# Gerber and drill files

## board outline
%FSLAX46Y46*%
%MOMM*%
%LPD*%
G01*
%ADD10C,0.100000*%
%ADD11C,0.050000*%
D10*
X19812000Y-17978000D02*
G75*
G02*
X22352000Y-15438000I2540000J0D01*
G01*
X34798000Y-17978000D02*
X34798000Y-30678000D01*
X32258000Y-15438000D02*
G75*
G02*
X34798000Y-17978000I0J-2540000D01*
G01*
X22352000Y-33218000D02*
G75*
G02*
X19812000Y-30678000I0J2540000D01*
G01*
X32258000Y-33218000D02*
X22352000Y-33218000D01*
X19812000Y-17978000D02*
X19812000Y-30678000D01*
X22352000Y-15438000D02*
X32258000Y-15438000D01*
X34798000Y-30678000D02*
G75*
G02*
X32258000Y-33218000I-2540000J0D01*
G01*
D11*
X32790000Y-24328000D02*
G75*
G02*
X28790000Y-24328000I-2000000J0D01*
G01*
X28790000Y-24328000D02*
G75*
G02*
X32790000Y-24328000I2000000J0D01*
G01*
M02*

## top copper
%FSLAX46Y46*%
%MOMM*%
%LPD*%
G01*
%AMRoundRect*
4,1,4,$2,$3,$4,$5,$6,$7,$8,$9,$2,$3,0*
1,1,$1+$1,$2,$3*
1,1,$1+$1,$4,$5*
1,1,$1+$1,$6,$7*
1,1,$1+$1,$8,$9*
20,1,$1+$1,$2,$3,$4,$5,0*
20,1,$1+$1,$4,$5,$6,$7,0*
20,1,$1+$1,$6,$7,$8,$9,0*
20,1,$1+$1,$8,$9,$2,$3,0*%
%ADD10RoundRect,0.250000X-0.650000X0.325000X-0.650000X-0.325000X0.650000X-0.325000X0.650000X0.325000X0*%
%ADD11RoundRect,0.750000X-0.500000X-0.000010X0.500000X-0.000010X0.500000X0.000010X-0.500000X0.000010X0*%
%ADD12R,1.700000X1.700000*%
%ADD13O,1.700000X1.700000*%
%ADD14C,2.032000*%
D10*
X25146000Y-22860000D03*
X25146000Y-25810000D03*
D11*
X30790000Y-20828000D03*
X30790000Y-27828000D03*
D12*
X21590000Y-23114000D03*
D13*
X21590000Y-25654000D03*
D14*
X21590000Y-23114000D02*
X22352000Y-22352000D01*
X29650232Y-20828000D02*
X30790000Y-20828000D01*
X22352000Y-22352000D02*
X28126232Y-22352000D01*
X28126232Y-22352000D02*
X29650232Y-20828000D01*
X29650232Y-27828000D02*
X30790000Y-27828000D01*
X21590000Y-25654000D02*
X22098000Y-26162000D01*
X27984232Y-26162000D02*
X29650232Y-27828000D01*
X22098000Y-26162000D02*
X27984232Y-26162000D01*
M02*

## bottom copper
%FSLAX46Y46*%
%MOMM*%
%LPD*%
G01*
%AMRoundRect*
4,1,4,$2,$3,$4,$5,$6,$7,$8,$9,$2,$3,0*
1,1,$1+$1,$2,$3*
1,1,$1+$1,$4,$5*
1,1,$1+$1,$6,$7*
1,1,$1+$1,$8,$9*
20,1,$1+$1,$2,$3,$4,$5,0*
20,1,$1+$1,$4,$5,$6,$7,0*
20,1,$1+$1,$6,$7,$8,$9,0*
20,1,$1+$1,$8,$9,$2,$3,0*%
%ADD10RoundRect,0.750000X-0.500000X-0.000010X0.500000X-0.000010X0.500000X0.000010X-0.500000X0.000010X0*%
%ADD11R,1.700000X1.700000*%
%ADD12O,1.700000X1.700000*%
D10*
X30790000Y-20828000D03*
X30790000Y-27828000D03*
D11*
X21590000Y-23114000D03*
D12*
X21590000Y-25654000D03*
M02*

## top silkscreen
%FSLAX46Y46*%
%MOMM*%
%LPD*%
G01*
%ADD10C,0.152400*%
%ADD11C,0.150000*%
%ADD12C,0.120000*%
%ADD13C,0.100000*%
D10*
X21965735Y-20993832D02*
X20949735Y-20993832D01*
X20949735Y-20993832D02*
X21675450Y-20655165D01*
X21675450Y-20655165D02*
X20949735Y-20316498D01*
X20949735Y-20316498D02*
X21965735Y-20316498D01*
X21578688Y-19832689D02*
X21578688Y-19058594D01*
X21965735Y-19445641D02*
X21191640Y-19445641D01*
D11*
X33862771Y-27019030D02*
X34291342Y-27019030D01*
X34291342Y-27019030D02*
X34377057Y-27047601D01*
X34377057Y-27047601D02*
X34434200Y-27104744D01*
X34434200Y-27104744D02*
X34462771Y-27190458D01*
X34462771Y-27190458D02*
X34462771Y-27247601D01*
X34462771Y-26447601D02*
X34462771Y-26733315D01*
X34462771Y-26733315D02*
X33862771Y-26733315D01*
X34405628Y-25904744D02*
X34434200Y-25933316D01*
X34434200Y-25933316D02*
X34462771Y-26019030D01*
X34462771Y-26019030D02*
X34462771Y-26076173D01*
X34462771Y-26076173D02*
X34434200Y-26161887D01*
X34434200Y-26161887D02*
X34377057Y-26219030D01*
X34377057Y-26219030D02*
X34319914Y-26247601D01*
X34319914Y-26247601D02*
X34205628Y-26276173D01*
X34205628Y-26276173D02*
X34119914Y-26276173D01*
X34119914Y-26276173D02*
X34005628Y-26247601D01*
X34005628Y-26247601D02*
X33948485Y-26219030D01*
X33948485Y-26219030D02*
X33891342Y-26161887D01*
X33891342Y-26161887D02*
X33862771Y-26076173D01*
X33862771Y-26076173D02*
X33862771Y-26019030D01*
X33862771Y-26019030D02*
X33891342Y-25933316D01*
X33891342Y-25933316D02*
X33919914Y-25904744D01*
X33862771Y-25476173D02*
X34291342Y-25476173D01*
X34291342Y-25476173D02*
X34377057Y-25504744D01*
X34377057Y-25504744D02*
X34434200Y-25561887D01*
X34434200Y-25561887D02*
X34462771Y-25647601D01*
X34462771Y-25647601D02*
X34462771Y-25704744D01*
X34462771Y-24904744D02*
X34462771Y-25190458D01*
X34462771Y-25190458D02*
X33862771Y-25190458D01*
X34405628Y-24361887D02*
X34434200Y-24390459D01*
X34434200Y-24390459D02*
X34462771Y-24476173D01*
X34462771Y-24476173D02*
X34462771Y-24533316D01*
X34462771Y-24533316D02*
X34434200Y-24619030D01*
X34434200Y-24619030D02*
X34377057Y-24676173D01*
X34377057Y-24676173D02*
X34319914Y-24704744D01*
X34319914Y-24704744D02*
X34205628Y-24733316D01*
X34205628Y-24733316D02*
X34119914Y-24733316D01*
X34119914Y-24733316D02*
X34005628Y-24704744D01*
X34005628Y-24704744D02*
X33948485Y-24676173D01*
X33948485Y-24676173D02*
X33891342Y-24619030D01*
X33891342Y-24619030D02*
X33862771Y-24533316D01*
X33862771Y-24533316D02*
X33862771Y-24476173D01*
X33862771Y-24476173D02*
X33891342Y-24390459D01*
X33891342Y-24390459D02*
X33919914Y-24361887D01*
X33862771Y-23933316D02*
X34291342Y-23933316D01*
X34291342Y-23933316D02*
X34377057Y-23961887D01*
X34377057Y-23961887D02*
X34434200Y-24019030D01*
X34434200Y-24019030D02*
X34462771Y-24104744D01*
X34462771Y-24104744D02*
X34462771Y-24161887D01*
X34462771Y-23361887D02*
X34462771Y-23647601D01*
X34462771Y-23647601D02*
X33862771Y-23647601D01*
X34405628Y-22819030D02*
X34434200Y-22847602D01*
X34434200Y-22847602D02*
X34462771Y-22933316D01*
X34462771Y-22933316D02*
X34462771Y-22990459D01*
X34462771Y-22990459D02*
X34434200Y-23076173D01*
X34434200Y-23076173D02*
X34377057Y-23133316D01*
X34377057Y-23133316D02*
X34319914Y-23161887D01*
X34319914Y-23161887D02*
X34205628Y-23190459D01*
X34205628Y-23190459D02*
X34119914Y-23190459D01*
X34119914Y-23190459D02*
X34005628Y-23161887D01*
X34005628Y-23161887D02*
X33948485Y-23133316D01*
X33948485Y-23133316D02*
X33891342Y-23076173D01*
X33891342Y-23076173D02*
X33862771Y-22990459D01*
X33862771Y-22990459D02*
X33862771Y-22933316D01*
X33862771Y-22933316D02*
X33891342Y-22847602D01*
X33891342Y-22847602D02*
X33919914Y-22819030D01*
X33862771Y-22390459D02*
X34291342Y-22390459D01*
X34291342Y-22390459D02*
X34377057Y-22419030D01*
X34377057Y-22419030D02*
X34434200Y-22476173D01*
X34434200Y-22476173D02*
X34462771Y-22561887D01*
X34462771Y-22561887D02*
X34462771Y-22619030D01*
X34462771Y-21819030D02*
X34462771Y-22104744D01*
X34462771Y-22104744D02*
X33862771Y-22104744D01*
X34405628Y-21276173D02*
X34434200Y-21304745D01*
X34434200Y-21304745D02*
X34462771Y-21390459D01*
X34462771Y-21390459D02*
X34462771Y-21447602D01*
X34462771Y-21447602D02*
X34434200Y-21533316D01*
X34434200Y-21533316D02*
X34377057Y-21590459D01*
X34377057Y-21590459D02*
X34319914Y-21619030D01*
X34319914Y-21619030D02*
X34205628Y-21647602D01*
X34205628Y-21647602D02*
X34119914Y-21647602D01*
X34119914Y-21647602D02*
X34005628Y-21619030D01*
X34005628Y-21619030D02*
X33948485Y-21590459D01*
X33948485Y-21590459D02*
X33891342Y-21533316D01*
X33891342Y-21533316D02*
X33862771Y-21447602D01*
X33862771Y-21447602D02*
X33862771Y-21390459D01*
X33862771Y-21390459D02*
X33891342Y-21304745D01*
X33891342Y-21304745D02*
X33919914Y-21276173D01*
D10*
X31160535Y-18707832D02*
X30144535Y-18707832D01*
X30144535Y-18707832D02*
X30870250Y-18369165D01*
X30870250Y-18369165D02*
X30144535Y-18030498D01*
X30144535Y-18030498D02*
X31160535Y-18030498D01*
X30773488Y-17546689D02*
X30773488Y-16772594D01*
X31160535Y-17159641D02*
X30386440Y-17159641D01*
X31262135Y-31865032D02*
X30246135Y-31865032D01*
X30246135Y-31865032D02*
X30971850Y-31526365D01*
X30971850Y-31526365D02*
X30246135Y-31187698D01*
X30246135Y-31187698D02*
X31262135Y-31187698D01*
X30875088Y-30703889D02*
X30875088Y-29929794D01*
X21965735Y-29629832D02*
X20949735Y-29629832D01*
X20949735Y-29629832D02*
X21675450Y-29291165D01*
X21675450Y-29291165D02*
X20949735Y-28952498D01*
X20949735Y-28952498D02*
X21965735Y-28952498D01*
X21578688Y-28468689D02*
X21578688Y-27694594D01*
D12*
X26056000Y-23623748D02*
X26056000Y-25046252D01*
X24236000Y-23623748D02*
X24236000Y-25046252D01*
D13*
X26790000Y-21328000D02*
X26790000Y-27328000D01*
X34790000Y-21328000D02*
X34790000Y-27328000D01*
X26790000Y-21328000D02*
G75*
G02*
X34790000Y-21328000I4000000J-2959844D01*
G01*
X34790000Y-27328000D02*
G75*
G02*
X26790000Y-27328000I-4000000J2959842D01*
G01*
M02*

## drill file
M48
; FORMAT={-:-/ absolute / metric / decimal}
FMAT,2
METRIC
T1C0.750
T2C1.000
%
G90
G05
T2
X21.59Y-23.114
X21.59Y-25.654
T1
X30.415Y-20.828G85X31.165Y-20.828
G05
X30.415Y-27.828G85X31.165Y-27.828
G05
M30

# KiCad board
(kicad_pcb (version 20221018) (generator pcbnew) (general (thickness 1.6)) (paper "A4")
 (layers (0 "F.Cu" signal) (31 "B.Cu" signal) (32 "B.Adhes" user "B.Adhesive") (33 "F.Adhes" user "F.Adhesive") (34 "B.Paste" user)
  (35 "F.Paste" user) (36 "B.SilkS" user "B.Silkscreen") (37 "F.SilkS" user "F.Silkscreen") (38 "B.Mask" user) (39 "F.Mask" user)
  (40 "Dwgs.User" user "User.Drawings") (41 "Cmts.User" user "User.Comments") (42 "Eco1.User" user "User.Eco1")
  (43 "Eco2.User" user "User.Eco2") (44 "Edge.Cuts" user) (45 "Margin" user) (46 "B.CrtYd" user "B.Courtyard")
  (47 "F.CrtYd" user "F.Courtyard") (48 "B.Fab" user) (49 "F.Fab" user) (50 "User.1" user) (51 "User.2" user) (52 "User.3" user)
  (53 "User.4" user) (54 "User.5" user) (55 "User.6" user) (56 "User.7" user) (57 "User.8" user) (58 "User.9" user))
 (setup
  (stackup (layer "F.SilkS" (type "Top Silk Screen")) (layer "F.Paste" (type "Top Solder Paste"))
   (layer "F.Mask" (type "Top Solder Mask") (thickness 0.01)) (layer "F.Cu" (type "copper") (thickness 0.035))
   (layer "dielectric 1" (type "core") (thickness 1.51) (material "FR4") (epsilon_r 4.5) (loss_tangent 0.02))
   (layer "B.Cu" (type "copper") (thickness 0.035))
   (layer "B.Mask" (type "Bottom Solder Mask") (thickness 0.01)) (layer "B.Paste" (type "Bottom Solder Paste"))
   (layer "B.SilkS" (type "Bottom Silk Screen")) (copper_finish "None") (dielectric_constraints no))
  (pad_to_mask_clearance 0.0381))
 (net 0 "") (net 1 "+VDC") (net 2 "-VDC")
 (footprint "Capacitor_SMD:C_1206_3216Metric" (layer "F.Cu") (at 25.146 24.335 -90)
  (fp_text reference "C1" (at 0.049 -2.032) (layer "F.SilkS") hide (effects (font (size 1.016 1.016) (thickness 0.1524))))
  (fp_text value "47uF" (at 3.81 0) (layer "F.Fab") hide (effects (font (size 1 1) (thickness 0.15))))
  (fp_line (start -0.711252 -0.91) (end 0.711252 -0.91) (stroke (width 0.12) (type solid)) (layer "F.SilkS"))
  (fp_line (start -0.711252 0.91) (end 0.711252 0.91) (stroke (width 0.12) (type solid)) (layer "F.SilkS"))
  (pad "1" smd roundrect (at -1.475 0 270) (size 1.15 1.8) (layers "F.Cu" "F.Paste" "F.Mask") (roundrect_rratio 0.2173913043) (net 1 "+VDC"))
  (pad "2" smd roundrect (at 1.475 0 270) (size 1.15 1.8) (layers "F.Cu" "F.Paste" "F.Mask") (roundrect_rratio 0.2173913043) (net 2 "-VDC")))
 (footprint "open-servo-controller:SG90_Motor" (layer "F.Cu") (at 30.79 24.328)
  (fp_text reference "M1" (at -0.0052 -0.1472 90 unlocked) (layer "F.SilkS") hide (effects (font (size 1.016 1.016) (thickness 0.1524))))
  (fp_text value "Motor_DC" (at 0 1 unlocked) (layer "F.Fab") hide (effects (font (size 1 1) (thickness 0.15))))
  (fp_line (start -4 -3) (end -4 3) (stroke (width 0.1) (type default)) (layer "F.SilkS"))
  (fp_line (start 4 -3) (end 4 3) (stroke (width 0.1) (type default)) (layer "F.SilkS"))
  (fp_arc (start -4 -3) (mid 0 -5.016166) (end 4 -3) (stroke (width 0.1) (type default)) (layer "F.SilkS"))
  (fp_arc (start 4 3) (mid 0 5.016167) (end -4 3) (stroke (width 0.1) (type default)) (layer "F.SilkS"))
  (fp_circle (center 0 0) (end 2 0) (stroke (width 0.05) (type default)) (fill none) (layer "Edge.Cuts"))
  (pad "1" thru_hole roundrect (at 0 -3.5) (size 2.5 1.5) (drill oval 1.5 0.75) (layers "*.Cu" "*.Mask") (roundrect_rratio 0.5)
   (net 1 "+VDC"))
  (pad "2" thru_hole roundrect (at 0 3.5) (size 2.5 1.5) (drill oval 1.5 0.75) (layers "*.Cu" "*.Mask") (roundrect_rratio 0.5)
   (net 2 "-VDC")))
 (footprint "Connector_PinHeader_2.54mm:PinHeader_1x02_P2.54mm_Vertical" (layer "B.Cu") (at 21.59 23.114 180)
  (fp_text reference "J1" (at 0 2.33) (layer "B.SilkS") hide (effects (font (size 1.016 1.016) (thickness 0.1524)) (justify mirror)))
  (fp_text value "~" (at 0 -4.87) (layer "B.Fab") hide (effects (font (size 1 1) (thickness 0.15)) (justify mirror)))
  (pad "1" thru_hole rect (at 0 0 180) (size 1.7 1.7) (drill 1) (layers "*.Cu" "*.Mask") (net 1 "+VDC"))
  (pad "2" thru_hole oval (at 0 -2.54 180) (size 1.7 1.7) (drill 1) (layers "*.Cu" "*.Mask") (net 2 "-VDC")))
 (gr_arc (start 19.812 17.978) (mid 20.555949 16.181949) (end 22.352 15.438) (stroke (width 0.1) (type default)) (layer "Edge.Cuts"))
 (gr_line (start 34.798 17.978) (end 34.798 30.678) (stroke (width 0.1) (type default)) (layer "Edge.Cuts"))
 (gr_arc (start 32.258 15.438) (mid 34.054051 16.181949) (end 34.798 17.978) (stroke (width 0.1) (type default)) (layer "Edge.Cuts"))
 (gr_arc (start 22.352 33.218) (mid 20.555949 32.474051) (end 19.812 30.678) (stroke (width 0.1) (type default)) (layer "Edge.Cuts"))
 (gr_line (start 32.258 33.218) (end 22.352 33.218) (stroke (width 0.1) (type default)) (layer "Edge.Cuts"))
 (gr_line (start 19.812 17.978) (end 19.812 30.678) (stroke (width 0.1) (type default)) (layer "Edge.Cuts"))
 (gr_line (start 22.352 15.438) (end 32.258 15.438) (stroke (width 0.1) (type default)) (layer "Edge.Cuts"))
 (gr_arc (start 34.798 30.678) (mid 34.054051 32.474051) (end 32.258 33.218) (stroke (width 0.1) (type default)) (layer "Edge.Cuts"))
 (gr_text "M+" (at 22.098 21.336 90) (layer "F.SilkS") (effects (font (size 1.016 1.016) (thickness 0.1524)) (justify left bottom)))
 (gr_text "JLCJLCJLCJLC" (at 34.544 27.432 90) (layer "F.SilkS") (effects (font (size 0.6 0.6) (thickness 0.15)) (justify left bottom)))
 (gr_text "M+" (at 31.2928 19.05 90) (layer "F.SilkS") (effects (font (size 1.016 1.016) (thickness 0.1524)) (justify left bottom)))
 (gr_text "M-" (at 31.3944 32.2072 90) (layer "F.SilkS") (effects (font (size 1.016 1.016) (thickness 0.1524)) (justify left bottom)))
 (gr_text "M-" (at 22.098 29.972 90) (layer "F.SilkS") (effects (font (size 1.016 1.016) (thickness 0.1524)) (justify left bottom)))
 (segment (start 21.59 23.114) (end 22.352 22.352) (width 2.032) (layer "F.Cu") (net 1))
 (segment (start 29.650232 20.828) (end 30.79 20.828) (width 2.032) (layer "F.Cu") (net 1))
 (segment (start 22.352 22.352) (end 28.126232 22.352) (width 2.032) (layer "F.Cu") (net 1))
 (segment (start 28.126232 22.352) (end 29.650232 20.828) (width 2.032) (layer "F.Cu") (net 1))
 (segment (start 29.650232 27.828) (end 30.79 27.828) (width 2.032) (layer "F.Cu") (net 2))
 (segment (start 21.59 25.654) (end 22.098 26.162) (width 2.032) (layer "F.Cu") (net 2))
 (segment (start 27.984232 26.162) (end 29.650232 27.828) (width 2.032) (layer "F.Cu") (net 2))
 (segment (start 22.098 26.162) (end 27.984232 26.162) (width 2.032) (layer "F.Cu") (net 2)))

